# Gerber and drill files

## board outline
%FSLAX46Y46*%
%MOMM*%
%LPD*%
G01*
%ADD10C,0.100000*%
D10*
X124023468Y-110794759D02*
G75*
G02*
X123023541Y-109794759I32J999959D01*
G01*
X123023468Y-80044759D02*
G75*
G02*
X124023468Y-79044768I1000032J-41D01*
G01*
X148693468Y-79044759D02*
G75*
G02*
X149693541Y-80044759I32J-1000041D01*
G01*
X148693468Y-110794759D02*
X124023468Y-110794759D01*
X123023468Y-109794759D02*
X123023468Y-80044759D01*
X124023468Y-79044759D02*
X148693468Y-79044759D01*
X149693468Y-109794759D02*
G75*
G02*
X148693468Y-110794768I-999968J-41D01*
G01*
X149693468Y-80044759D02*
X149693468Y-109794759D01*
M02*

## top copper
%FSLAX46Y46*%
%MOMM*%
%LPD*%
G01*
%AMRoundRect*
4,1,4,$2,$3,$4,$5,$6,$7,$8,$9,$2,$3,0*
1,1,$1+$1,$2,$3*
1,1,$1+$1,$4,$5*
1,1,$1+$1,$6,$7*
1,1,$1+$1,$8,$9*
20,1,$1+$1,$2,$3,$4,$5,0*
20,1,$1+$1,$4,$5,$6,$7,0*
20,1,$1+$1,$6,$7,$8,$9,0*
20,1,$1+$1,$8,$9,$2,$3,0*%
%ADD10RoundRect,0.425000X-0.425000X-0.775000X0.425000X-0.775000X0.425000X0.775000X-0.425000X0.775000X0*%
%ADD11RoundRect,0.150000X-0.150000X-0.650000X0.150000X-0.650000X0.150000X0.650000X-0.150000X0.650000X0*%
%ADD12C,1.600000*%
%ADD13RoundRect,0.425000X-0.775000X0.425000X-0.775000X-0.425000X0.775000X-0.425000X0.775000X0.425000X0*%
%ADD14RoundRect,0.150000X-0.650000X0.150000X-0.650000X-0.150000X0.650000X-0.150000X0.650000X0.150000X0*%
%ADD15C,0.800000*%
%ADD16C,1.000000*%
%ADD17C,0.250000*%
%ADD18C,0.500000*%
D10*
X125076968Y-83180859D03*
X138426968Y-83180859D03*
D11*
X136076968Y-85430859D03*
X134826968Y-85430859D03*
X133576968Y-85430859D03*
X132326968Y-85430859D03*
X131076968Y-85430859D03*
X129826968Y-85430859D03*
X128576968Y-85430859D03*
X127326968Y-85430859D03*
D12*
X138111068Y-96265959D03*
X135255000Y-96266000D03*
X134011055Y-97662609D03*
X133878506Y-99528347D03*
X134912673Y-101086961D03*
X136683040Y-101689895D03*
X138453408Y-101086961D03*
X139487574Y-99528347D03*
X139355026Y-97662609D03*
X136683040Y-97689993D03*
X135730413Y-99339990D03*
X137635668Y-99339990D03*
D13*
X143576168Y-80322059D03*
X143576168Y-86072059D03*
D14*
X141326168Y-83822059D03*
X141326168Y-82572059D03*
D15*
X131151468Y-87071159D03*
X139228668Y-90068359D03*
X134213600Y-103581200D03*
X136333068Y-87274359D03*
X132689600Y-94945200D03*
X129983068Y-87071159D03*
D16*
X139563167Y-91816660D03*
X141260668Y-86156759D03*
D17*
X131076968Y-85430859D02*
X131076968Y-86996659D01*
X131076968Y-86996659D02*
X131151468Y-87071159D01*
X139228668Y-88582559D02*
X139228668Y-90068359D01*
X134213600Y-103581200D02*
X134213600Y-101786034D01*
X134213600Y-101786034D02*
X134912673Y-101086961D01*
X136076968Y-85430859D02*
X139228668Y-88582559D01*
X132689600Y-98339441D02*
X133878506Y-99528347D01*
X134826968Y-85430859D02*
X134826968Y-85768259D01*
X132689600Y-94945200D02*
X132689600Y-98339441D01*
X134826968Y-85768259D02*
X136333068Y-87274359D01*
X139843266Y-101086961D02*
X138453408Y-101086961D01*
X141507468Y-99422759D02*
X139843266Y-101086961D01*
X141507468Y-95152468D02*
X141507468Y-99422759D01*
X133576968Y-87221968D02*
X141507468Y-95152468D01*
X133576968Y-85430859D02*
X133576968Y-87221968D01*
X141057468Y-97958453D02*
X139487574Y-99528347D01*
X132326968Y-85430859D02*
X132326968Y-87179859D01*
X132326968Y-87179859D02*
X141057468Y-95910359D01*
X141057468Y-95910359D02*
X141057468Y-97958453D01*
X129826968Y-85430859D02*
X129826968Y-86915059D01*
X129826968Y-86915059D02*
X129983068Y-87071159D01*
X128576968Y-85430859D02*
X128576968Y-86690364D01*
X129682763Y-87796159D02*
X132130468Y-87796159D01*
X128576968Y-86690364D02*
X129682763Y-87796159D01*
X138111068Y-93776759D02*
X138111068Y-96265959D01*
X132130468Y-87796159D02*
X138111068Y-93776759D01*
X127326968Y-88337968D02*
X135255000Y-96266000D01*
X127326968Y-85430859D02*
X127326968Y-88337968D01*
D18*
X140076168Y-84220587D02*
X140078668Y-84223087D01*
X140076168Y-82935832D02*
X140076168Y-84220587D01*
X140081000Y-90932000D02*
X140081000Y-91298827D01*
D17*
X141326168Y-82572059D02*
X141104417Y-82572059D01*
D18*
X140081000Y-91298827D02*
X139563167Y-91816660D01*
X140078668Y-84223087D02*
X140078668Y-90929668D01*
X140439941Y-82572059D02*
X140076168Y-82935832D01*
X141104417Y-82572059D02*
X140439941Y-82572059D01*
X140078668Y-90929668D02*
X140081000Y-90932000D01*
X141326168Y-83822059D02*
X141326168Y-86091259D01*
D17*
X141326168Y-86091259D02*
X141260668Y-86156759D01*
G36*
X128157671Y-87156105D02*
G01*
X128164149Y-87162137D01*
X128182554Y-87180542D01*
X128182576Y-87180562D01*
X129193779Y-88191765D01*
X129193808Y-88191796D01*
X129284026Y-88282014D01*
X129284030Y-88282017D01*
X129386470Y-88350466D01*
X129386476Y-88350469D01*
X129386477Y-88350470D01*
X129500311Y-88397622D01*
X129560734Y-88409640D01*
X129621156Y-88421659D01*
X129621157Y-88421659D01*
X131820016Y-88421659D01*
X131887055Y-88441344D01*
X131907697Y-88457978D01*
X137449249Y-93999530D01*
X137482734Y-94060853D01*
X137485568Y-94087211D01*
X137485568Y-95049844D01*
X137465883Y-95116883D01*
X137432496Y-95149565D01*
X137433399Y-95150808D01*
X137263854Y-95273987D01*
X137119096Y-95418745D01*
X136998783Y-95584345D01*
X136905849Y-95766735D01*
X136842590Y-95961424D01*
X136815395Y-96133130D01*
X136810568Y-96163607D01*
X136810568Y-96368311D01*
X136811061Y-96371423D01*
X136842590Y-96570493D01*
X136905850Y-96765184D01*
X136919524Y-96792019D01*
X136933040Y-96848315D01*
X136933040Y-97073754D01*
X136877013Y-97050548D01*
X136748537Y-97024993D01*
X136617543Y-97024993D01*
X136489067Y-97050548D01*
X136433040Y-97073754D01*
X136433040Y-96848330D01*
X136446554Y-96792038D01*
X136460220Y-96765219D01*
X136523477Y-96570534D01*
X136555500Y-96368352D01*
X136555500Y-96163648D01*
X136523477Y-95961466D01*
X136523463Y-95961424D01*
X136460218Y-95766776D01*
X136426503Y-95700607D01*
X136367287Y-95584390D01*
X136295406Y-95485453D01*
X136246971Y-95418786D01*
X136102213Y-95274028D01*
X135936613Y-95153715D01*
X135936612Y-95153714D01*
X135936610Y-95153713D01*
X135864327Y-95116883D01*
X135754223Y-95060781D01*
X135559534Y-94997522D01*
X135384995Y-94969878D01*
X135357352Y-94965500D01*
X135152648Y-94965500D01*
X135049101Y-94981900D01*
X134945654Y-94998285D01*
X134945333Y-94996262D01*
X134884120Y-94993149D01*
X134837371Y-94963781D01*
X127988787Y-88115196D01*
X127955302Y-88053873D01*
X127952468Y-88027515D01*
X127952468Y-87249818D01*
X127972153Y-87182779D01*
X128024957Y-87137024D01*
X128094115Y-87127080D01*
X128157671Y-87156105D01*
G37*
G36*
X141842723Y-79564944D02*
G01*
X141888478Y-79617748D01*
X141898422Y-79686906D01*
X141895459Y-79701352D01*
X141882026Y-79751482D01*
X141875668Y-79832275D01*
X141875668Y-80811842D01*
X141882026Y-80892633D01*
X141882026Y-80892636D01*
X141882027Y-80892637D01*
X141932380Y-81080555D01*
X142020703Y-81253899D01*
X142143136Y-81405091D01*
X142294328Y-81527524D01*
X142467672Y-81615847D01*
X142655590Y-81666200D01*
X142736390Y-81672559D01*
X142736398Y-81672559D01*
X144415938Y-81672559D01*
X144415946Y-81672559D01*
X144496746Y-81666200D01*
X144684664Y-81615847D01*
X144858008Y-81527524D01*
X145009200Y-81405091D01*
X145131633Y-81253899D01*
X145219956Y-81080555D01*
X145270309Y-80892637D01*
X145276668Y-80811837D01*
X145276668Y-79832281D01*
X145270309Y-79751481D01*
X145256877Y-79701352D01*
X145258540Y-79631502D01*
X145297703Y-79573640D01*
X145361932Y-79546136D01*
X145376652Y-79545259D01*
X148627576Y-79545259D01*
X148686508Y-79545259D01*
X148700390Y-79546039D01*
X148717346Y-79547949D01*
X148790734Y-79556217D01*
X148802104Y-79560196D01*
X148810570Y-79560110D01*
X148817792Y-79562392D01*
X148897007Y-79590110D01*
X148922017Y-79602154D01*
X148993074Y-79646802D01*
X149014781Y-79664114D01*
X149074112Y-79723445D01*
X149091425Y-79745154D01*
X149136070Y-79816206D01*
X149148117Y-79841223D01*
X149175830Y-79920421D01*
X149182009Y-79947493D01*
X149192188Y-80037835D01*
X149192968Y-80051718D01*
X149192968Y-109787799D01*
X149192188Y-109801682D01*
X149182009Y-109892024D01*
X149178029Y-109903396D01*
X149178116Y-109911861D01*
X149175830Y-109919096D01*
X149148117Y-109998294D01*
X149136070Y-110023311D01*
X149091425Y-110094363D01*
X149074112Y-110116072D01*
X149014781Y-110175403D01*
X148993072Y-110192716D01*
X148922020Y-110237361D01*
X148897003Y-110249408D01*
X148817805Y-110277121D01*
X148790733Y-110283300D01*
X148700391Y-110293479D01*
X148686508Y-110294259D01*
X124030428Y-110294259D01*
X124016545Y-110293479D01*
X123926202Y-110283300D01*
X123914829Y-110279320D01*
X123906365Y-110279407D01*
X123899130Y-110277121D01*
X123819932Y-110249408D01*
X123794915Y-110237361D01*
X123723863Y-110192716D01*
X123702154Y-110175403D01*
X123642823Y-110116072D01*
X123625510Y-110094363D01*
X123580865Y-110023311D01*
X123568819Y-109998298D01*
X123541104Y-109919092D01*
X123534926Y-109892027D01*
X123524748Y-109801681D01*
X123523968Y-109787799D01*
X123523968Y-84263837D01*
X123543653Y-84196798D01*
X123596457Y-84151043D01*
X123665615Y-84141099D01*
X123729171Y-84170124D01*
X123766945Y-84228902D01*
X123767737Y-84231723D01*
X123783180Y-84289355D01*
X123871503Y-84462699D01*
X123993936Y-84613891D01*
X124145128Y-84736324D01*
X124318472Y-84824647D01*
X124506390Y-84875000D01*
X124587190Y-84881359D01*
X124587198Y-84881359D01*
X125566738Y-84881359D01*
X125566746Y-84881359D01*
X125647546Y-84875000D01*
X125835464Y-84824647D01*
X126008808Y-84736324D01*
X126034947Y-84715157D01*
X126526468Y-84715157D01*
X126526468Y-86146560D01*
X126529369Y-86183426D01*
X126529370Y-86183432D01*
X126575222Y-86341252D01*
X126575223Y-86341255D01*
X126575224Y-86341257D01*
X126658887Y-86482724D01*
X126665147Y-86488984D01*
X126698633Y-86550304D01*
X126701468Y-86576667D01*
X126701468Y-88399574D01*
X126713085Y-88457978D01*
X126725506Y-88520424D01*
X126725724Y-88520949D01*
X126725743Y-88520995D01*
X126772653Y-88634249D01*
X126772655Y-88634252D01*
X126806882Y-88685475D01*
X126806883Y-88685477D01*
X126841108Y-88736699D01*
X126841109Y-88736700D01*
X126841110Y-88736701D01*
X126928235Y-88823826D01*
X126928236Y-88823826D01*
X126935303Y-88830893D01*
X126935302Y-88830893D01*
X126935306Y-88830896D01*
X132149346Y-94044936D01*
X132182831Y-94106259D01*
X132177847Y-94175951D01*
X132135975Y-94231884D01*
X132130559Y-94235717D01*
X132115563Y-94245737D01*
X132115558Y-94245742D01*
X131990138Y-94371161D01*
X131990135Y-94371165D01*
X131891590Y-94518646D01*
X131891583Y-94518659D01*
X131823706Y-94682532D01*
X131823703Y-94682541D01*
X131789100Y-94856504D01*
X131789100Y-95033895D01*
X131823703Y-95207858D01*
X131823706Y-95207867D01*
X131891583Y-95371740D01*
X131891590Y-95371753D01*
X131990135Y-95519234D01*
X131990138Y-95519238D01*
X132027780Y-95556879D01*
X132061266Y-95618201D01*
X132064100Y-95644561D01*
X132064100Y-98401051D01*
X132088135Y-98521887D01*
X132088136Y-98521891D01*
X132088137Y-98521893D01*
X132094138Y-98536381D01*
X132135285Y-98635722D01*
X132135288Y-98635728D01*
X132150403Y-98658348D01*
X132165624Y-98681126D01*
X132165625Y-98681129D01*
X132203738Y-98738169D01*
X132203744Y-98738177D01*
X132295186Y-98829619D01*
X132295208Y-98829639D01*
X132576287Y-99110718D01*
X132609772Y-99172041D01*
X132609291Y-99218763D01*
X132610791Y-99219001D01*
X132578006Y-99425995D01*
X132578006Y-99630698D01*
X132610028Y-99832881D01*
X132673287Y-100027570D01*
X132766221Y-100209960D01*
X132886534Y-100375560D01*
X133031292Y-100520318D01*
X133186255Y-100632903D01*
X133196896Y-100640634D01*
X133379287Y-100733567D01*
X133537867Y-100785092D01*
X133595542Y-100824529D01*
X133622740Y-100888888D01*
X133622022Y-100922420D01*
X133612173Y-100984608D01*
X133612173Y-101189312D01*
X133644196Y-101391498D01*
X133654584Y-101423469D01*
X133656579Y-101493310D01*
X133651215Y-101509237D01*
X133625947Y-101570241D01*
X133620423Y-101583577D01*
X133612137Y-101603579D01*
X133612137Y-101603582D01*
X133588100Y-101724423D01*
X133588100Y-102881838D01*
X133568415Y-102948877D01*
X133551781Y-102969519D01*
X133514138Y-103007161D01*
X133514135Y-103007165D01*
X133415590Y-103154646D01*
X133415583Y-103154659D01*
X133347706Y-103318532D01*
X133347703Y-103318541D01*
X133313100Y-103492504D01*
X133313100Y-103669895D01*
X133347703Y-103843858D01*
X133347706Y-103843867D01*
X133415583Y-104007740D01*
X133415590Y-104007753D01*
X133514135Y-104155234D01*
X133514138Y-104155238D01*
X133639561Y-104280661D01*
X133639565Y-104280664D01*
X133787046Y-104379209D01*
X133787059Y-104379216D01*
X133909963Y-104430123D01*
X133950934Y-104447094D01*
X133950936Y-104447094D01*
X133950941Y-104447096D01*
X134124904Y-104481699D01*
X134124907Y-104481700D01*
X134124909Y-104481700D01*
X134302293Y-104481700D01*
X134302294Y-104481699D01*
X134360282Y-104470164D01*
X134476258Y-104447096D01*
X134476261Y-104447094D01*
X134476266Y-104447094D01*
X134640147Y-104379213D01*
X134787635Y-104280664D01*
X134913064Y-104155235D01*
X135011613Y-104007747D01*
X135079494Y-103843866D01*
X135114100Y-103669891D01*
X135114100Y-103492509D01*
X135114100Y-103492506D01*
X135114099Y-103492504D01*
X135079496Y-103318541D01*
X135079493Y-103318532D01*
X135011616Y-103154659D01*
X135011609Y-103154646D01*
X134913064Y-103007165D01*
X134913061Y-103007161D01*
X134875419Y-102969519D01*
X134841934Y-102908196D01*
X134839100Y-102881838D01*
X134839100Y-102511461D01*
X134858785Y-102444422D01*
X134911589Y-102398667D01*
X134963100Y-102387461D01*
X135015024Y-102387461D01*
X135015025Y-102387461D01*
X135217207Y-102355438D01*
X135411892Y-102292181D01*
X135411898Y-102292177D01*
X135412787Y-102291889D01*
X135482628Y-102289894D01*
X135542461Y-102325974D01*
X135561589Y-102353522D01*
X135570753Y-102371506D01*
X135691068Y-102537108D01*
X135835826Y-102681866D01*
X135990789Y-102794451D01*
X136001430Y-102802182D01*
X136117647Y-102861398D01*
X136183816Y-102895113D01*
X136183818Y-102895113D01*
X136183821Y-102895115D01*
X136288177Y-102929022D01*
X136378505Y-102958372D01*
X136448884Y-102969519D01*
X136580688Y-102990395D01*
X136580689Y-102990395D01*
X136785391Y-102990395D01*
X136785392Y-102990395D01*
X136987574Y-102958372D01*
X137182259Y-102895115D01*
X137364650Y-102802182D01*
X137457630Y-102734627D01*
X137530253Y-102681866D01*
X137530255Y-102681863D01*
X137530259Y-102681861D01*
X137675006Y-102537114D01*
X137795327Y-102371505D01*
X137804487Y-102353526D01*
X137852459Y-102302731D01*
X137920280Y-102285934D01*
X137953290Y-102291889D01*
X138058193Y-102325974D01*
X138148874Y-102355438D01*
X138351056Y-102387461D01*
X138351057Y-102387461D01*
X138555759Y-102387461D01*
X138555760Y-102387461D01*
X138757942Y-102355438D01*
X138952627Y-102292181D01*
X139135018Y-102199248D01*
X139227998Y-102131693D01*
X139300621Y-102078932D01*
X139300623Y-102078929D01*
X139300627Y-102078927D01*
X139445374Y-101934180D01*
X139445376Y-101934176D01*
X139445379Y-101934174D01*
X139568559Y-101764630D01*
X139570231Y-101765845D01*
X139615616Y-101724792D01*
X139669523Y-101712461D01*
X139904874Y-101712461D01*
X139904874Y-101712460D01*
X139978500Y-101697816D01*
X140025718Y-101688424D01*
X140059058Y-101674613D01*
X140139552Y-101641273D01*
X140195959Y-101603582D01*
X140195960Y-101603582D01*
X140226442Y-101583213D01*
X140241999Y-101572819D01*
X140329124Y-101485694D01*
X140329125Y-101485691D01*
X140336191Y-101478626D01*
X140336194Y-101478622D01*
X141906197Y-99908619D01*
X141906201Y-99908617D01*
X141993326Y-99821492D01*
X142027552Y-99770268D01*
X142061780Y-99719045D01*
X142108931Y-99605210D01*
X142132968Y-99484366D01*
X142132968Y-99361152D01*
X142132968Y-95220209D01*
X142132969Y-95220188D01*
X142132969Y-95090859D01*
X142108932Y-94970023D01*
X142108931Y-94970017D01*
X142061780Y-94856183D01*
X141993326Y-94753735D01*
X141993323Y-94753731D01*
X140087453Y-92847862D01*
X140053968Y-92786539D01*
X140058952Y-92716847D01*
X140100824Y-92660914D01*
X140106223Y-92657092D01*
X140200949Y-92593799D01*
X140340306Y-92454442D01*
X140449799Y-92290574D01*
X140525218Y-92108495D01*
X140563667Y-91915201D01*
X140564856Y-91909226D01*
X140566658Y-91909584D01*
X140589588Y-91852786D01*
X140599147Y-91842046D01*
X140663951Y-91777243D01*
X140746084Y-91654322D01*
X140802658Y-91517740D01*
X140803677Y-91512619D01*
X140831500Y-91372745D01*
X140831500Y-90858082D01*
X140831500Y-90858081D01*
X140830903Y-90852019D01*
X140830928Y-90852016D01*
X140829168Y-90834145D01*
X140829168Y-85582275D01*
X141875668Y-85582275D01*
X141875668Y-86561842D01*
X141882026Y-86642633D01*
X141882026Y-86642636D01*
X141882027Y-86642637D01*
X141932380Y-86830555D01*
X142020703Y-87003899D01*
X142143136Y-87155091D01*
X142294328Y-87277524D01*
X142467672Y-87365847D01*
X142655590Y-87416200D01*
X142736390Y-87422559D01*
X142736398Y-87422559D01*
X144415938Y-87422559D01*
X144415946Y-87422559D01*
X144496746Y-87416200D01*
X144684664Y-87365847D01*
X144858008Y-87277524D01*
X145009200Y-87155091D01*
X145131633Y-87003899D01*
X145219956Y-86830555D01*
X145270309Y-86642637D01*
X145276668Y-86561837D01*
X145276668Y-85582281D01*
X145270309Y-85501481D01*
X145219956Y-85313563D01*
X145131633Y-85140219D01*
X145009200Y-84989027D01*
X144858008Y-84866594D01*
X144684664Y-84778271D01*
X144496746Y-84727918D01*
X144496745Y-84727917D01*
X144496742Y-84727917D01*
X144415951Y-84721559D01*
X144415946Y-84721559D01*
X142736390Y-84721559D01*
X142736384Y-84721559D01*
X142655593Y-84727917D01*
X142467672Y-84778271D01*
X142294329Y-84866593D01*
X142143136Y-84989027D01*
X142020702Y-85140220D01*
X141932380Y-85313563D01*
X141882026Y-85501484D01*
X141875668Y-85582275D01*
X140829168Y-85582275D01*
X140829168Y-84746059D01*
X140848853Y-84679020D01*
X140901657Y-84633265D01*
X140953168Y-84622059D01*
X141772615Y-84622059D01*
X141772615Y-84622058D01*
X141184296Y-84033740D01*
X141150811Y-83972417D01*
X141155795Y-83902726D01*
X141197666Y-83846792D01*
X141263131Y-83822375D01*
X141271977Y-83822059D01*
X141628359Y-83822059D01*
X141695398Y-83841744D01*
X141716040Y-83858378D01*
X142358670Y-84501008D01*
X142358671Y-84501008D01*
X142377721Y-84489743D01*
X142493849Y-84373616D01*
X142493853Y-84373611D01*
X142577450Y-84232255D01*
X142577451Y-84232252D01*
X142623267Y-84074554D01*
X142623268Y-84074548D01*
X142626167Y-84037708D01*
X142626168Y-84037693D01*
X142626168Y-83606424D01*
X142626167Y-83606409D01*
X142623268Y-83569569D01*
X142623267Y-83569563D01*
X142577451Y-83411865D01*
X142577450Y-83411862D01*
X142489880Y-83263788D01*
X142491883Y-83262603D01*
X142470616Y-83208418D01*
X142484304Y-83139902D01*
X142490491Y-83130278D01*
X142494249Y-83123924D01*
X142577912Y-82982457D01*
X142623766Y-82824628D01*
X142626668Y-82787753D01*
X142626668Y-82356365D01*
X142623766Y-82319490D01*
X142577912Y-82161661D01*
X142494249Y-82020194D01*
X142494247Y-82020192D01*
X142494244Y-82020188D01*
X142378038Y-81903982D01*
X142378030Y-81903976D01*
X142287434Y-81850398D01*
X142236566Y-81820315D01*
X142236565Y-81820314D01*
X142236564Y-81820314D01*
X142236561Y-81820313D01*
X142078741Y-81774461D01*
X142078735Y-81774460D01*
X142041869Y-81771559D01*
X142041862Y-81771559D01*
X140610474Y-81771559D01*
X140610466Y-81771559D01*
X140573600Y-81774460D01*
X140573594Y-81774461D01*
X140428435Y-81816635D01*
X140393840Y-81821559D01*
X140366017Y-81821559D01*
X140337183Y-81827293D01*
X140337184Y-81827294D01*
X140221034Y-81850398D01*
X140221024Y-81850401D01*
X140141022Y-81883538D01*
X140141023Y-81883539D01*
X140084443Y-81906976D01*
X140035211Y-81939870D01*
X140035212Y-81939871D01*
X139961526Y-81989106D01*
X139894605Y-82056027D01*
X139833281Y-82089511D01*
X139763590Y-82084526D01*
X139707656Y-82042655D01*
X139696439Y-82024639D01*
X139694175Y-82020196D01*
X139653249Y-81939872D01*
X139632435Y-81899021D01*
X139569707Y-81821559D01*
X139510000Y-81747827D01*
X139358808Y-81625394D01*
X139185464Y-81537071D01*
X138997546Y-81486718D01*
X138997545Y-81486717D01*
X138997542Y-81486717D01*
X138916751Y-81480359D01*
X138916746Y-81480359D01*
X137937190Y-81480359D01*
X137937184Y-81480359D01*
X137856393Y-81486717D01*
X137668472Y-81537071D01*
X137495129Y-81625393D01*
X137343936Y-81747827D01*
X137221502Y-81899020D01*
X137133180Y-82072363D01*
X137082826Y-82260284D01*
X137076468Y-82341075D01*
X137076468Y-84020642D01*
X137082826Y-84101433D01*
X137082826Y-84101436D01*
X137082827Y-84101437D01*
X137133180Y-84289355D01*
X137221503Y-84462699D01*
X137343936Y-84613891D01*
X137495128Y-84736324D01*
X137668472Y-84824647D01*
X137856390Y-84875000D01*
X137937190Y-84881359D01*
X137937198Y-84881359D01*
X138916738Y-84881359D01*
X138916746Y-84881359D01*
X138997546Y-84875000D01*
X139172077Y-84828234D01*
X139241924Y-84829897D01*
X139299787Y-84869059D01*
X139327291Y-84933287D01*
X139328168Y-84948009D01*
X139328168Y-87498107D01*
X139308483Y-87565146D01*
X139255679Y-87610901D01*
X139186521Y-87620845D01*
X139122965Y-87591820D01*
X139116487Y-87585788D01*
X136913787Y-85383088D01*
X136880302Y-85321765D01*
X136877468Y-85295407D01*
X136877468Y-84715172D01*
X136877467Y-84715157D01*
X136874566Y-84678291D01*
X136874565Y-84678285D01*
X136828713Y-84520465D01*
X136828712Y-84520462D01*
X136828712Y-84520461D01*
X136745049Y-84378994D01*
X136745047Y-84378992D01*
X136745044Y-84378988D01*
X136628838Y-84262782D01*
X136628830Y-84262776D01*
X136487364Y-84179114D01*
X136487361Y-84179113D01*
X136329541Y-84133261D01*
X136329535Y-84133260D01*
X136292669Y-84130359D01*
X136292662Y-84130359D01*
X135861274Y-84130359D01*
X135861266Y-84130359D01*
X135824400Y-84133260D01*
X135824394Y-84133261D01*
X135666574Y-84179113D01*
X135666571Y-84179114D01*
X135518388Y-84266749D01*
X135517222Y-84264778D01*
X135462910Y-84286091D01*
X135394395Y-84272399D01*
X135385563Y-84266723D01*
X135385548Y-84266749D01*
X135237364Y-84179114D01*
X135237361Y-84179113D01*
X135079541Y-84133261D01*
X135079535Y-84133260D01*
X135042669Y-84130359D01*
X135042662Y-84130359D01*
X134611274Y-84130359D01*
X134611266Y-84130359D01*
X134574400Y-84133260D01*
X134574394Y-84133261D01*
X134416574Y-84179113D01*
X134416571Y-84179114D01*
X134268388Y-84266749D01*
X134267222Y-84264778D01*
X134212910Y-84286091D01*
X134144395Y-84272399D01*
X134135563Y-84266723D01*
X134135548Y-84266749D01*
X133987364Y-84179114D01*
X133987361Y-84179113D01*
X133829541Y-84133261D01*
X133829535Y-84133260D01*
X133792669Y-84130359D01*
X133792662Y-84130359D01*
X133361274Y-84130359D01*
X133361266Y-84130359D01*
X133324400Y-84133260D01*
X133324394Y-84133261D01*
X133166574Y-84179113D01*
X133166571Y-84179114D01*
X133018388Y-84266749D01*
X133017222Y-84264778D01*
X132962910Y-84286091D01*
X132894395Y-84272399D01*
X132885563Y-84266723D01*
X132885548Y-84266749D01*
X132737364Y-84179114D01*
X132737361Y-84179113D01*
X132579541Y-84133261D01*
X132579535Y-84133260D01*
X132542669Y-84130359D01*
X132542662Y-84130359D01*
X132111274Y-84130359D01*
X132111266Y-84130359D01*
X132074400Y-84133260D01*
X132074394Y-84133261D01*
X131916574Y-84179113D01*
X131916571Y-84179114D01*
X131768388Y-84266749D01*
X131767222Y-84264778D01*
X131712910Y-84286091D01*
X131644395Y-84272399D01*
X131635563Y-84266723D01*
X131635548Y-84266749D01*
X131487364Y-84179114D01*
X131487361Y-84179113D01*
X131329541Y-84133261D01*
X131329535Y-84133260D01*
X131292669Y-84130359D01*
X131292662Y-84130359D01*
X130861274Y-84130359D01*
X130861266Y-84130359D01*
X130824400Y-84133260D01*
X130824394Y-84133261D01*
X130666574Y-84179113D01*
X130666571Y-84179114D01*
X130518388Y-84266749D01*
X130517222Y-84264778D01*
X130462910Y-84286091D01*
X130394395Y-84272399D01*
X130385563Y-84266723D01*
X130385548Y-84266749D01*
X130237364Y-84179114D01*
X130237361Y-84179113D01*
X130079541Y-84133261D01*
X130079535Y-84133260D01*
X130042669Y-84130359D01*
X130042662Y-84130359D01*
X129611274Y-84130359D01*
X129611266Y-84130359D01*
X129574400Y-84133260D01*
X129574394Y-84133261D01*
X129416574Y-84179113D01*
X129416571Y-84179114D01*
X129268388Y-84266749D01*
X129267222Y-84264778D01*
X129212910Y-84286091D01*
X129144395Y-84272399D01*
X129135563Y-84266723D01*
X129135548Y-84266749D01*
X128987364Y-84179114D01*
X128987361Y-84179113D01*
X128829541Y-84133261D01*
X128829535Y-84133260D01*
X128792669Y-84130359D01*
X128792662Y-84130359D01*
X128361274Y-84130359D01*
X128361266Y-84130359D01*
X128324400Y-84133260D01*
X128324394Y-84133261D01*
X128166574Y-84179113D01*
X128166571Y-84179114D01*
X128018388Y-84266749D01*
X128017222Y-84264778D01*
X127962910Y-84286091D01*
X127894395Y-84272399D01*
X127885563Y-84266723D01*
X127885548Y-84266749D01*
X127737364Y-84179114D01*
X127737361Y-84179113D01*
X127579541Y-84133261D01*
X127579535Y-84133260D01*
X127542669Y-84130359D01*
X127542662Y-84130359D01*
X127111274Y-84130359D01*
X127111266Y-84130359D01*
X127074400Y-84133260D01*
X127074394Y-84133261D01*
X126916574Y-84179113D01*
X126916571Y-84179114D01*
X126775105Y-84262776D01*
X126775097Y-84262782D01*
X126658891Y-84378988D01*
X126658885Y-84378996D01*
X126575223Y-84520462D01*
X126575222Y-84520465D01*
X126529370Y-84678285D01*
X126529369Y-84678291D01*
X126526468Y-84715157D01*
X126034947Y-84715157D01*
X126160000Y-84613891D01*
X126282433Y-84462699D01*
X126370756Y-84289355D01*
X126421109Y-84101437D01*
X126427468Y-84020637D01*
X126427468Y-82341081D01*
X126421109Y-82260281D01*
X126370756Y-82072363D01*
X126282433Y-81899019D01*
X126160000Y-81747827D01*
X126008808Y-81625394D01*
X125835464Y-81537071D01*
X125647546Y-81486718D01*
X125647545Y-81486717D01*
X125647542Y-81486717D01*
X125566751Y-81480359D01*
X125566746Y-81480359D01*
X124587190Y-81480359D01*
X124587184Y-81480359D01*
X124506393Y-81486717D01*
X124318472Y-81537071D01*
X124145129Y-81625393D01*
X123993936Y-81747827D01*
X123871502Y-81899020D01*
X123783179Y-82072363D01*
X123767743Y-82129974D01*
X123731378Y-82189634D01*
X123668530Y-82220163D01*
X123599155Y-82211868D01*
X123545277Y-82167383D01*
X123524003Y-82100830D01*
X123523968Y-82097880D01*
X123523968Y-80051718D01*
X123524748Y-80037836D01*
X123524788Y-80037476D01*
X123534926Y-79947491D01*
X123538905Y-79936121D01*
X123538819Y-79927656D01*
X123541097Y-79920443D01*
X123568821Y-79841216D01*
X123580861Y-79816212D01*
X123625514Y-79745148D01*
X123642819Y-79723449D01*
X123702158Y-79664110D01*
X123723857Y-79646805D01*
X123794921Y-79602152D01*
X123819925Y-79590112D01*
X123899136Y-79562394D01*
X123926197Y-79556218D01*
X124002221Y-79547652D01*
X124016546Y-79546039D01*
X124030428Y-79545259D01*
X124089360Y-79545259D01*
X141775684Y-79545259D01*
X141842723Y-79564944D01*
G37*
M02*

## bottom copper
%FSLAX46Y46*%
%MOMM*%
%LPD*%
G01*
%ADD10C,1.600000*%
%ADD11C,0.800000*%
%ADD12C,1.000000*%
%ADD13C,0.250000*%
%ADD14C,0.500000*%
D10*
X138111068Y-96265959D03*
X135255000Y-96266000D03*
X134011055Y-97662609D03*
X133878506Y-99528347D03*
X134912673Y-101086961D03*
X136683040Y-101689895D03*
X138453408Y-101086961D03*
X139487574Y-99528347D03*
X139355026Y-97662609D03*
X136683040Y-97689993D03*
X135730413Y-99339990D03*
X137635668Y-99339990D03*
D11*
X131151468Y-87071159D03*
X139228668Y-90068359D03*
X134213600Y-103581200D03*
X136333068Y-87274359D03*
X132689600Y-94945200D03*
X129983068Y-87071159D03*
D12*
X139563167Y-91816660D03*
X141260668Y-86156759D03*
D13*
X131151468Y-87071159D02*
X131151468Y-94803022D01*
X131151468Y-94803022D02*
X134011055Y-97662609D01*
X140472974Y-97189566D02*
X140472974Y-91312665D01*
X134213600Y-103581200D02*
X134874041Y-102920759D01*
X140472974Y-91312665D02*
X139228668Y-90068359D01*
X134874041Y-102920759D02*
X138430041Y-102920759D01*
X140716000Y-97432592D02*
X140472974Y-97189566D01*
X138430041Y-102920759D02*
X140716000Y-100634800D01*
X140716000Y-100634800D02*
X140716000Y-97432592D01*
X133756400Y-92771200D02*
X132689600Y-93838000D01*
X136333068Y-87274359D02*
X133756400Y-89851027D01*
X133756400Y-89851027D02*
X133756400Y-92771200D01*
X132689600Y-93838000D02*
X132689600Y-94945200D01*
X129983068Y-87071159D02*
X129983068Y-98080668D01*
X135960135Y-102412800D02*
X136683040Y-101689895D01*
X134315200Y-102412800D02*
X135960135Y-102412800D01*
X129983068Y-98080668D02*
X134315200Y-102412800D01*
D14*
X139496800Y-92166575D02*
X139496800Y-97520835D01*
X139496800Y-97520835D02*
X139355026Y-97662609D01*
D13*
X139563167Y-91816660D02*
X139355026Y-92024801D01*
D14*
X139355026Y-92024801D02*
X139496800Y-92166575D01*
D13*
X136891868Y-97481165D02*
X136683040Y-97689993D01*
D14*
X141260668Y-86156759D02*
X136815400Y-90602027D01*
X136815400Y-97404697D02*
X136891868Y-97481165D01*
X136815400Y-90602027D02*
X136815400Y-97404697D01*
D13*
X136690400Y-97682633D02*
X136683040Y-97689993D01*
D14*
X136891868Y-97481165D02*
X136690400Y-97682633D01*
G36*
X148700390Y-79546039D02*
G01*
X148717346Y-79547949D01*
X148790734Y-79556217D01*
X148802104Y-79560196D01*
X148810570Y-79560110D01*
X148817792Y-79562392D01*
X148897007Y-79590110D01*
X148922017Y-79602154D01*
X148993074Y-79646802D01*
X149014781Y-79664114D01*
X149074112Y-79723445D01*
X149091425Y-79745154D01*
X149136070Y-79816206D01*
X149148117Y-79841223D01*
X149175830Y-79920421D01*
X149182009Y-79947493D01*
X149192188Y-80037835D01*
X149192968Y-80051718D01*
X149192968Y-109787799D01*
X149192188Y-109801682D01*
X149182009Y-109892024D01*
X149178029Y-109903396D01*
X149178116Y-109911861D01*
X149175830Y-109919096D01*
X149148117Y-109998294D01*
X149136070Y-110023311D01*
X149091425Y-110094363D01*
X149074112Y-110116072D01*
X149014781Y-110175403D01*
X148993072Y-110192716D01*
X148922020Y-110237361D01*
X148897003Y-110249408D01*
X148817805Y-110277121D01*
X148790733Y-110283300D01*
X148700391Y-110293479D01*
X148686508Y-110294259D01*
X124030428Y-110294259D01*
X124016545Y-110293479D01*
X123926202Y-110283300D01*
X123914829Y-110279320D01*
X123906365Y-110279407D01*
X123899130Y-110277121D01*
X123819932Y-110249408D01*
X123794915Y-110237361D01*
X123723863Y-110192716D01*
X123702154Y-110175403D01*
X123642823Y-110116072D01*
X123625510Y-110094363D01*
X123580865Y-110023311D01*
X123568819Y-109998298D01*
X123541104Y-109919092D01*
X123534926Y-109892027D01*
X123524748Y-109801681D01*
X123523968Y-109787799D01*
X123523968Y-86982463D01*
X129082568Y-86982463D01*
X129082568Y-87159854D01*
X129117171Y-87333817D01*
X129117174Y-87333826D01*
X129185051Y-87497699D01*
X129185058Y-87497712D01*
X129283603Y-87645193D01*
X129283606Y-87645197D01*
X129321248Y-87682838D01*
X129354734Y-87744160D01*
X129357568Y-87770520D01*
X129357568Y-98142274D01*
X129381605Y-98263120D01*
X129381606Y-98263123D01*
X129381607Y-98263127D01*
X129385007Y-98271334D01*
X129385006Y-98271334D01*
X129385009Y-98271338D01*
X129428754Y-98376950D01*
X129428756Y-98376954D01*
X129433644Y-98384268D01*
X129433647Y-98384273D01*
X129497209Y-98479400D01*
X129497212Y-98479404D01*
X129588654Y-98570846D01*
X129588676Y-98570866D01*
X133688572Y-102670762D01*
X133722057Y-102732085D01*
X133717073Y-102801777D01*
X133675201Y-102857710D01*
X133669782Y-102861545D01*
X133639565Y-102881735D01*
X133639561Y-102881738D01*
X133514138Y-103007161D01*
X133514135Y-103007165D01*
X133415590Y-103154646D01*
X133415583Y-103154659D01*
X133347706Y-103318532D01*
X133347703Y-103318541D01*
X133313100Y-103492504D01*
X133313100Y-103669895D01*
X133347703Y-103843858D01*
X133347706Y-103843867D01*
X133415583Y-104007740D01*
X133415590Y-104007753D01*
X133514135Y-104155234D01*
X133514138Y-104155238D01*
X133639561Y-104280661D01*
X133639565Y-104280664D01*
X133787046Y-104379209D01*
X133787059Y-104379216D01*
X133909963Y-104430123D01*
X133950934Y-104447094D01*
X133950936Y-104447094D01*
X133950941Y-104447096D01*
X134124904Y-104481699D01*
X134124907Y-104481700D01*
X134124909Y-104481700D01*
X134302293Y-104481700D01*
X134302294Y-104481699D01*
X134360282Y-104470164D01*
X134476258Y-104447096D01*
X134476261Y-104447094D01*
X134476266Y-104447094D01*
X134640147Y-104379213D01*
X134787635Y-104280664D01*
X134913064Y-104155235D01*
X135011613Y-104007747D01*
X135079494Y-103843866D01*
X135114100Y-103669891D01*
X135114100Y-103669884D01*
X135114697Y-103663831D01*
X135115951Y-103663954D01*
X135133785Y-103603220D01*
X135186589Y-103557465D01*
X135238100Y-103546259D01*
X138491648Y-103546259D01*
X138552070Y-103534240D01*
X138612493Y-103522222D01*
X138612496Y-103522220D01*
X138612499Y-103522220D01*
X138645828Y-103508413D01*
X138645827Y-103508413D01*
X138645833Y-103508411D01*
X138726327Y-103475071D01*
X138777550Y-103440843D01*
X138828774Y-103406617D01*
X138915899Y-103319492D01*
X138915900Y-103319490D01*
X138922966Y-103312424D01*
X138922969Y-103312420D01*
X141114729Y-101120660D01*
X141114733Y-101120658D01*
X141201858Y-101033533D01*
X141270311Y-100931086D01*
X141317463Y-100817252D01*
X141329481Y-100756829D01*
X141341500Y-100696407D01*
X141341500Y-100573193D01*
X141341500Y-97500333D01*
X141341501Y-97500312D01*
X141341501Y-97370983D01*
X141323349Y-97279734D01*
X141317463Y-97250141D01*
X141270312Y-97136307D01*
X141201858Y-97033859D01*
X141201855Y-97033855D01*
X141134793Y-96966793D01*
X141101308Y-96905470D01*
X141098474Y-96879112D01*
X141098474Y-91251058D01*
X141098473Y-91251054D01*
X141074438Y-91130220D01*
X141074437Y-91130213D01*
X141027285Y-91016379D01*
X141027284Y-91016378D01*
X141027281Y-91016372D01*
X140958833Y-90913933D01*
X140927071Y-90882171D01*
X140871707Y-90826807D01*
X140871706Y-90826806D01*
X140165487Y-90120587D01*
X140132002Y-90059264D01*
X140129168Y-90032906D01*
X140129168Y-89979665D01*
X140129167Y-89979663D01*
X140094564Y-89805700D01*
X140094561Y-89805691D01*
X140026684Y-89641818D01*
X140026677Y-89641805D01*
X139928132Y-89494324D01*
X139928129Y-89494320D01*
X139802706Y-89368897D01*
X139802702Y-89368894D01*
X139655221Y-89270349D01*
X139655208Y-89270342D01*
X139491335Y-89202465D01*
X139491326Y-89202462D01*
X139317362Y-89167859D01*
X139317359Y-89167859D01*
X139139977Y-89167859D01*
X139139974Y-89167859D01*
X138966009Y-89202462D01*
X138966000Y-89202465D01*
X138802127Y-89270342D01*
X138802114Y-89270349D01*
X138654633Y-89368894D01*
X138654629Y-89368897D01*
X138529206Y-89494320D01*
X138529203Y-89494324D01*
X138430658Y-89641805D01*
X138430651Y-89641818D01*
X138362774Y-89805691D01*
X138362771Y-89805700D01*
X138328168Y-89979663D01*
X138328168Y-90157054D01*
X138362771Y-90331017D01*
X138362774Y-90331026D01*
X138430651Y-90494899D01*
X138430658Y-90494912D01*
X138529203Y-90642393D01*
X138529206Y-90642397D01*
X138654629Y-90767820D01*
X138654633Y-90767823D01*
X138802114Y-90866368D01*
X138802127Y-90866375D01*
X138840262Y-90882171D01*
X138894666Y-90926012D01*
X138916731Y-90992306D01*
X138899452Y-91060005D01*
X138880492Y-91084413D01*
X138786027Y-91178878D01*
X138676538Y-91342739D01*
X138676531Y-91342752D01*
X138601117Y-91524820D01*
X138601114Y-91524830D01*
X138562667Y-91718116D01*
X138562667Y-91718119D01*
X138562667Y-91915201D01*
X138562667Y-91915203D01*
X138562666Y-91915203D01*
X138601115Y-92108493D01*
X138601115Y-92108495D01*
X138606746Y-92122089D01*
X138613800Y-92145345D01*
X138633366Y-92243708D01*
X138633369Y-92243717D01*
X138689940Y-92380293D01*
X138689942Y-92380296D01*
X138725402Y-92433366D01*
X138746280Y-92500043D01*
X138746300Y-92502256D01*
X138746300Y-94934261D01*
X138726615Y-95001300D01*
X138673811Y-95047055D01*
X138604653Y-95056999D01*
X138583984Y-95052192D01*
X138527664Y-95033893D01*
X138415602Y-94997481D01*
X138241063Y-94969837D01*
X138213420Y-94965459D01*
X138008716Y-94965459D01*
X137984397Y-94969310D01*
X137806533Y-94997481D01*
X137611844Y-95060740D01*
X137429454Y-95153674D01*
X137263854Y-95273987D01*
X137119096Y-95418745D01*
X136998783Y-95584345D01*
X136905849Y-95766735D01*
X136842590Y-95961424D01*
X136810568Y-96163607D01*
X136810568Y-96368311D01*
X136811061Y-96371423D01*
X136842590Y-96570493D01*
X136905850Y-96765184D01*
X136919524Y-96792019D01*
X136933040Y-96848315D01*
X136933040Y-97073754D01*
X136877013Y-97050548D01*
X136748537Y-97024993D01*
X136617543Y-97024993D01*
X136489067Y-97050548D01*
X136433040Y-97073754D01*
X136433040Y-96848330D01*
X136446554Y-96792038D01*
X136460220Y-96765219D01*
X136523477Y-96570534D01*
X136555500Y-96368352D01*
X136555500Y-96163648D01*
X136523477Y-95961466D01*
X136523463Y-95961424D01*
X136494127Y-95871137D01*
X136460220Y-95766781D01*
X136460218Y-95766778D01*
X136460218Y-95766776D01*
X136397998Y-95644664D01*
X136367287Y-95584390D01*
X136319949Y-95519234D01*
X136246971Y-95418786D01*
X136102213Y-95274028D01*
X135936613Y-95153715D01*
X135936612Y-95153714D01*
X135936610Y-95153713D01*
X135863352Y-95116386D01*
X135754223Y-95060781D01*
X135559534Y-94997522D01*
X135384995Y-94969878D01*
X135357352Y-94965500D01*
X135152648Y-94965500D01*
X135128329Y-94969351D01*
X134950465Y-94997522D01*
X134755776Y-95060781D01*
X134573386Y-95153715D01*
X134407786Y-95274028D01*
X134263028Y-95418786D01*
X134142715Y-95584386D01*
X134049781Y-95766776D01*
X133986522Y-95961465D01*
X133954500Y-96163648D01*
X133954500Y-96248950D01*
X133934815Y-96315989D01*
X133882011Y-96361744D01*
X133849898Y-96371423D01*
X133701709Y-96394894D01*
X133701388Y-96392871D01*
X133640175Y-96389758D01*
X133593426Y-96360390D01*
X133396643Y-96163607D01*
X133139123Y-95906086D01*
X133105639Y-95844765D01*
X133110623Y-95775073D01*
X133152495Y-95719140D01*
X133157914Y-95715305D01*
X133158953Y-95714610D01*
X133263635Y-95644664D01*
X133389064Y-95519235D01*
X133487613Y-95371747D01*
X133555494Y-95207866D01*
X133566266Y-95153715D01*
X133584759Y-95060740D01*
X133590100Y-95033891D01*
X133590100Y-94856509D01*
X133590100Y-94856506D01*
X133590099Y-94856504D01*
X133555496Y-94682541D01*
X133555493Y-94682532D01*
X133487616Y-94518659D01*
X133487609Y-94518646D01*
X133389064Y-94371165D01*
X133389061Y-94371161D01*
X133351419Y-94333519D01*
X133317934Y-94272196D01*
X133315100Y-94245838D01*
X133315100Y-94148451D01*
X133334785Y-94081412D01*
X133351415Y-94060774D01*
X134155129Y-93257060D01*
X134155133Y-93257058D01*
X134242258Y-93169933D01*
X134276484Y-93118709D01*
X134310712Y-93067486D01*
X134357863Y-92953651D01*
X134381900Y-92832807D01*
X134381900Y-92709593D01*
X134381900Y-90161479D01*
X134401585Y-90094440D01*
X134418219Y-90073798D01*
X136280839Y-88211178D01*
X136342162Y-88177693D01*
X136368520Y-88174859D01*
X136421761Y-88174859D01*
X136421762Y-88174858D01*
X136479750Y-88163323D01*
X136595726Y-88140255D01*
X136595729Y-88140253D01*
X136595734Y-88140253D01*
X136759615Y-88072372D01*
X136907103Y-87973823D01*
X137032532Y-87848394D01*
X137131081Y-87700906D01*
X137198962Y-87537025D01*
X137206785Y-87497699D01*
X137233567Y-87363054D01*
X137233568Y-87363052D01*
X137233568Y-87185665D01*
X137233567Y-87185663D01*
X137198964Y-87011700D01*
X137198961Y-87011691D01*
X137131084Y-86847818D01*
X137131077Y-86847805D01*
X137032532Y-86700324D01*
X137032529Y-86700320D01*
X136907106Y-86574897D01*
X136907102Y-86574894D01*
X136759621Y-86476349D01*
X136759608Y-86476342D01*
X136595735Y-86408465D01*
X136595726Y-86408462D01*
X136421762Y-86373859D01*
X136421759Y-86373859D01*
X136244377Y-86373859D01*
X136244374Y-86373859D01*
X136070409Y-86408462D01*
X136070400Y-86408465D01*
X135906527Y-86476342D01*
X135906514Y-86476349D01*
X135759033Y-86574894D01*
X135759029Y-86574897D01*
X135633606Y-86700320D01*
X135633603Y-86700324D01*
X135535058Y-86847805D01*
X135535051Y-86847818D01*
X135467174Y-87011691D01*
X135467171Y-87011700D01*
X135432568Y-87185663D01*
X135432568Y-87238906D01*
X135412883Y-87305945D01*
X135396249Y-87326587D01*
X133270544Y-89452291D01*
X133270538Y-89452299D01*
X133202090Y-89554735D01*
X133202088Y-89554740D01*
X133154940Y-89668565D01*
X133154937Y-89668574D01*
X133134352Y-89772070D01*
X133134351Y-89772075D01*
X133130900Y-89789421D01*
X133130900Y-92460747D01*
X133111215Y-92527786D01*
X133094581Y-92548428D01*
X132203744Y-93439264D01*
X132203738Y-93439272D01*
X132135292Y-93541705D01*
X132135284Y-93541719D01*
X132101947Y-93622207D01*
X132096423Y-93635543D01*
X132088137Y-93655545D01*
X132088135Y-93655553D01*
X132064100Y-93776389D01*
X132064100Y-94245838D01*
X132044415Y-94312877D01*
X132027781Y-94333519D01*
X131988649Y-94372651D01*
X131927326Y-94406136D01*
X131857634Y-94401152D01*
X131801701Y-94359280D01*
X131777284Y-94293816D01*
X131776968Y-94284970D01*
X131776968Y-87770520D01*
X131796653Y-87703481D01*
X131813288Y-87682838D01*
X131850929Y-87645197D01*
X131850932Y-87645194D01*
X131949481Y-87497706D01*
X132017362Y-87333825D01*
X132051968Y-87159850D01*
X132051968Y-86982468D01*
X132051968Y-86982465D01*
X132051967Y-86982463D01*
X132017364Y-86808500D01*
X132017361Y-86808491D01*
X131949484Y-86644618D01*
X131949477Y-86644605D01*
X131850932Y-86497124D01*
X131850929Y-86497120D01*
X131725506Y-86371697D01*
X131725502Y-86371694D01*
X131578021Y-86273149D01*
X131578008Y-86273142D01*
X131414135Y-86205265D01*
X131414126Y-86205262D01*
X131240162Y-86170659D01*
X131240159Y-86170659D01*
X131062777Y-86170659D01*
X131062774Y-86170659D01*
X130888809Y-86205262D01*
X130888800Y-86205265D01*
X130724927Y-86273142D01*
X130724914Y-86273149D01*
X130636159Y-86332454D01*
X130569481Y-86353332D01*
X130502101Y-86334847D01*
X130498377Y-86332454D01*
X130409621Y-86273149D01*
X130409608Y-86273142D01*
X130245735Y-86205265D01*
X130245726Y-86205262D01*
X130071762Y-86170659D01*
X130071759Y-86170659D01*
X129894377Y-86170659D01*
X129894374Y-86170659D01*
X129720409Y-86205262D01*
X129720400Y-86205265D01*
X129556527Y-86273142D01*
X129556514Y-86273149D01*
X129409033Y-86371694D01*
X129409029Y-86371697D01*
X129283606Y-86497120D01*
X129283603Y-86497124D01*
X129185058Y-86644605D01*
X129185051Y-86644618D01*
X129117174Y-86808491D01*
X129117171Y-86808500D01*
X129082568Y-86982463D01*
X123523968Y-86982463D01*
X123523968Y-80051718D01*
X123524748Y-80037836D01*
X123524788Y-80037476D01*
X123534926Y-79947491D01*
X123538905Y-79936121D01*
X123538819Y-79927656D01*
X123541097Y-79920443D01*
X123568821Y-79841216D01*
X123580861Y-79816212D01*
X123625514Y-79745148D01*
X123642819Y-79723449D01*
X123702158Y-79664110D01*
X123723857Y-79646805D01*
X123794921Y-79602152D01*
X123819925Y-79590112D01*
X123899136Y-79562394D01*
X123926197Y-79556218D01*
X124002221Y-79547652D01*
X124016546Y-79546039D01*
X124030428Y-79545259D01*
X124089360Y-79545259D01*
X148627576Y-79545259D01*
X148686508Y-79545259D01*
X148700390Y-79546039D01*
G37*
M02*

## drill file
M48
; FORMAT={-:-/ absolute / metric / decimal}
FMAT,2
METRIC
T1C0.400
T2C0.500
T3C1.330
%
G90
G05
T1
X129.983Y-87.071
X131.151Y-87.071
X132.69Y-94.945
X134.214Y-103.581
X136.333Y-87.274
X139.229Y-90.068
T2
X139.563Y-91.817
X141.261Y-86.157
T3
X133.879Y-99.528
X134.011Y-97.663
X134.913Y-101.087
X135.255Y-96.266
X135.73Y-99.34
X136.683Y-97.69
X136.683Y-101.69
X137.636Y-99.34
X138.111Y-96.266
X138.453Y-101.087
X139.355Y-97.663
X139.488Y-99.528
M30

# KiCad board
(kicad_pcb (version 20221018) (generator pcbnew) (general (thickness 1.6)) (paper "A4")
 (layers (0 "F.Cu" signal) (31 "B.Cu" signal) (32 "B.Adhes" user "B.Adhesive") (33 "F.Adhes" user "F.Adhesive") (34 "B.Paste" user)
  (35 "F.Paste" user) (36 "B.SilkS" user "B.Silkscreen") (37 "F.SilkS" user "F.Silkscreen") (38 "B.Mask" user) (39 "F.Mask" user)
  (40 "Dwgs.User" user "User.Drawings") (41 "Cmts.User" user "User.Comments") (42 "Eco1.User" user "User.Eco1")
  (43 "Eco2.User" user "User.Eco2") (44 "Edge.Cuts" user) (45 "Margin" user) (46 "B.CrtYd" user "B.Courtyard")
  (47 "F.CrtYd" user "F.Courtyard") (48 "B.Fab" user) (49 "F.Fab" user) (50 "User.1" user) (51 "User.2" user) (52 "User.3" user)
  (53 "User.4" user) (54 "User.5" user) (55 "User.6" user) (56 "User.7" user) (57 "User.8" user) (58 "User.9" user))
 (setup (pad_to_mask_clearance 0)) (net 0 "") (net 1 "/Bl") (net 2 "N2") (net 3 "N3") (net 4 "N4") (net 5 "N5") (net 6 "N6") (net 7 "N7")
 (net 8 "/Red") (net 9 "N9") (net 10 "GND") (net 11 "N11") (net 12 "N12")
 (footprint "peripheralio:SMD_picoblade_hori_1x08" (layer "F.Cu") (at 124.226968 86.230859)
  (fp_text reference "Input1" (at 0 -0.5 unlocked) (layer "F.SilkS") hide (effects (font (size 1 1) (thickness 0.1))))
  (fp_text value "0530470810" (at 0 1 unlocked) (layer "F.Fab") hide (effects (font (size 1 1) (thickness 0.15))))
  (pad "" smd roundrect (at 0.85 -3.05) (size 1.7 2.4) (layers "F.Cu" "F.Paste" "F.Mask") (roundrect_rratio 0.25) (thermal_bridge_angle 45))
  (pad "" smd roundrect (at 14.2 -3.05) (size 1.7 2.4) (layers "F.Cu" "F.Paste" "F.Mask") (roundrect_rratio 0.25) (thermal_bridge_angle 45))
  (pad "1" smd roundrect (at 11.85 -0.8) (size 0.6 1.6) (layers "F.Cu" "F.Paste" "F.Mask") (roundrect_rratio 0.25) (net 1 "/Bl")
   (thermal_bridge_angle 45))
  (pad "2" smd roundrect (at 10.6 -0.8) (size 0.6 1.6) (layers "F.Cu" "F.Paste" "F.Mask") (roundrect_rratio 0.25) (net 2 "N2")
   (thermal_bridge_angle 45))
  (pad "3" smd roundrect (at 9.35 -0.8) (size 0.6 1.6) (layers "F.Cu" "F.Paste" "F.Mask") (roundrect_rratio 0.25) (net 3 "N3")
   (thermal_bridge_angle 45))
  (pad "4" smd roundrect (at 8.1 -0.8) (size 0.6 1.6) (layers "F.Cu" "F.Paste" "F.Mask") (roundrect_rratio 0.25) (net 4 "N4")
   (thermal_bridge_angle 45))
  (pad "5" smd roundrect (at 6.85 -0.8) (size 0.6 1.6) (layers "F.Cu" "F.Paste" "F.Mask") (roundrect_rratio 0.25) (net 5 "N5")
   (thermal_bridge_angle 45))
  (pad "6" smd roundrect (at 5.6 -0.8) (size 0.6 1.6) (layers "F.Cu" "F.Paste" "F.Mask") (roundrect_rratio 0.25) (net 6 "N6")
   (thermal_bridge_angle 45))
  (pad "7" smd roundrect (at 4.35 -0.8) (size 0.6 1.6) (layers "F.Cu" "F.Paste" "F.Mask") (roundrect_rratio 0.25) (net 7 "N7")
   (thermal_bridge_angle 45))
  (pad "8" smd roundrect (at 3.1 -0.8) (size 0.6 1.6) (layers "F.Cu" "F.Paste" "F.Mask") (roundrect_rratio 0.25) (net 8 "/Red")
   (thermal_bridge_angle 45)))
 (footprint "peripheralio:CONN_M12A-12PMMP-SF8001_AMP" (layer "F.Cu") (at 138.111068 96.265959 45)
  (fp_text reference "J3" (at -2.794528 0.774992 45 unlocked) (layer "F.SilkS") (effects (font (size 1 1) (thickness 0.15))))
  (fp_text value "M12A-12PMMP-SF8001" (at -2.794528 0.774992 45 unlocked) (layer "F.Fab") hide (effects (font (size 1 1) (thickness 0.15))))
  (pad "1" thru_hole circle (at 0 0 45) (size 1.6 1.6) (drill 1.33) (layers "*.Cu" "*.Mask") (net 7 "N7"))
  (pad "2" thru_hole circle (at -2.019574 -2.019516 45) (size 1.6 1.6) (drill 1.33) (layers "*.Cu" "*.Mask") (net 8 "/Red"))
  (pad "3" thru_hole circle (at -3.886728 -1.911566 135) (size 1.6 1.6) (drill 1.33) (layers "*.Cu" "*.Mask") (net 5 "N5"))
  (pad "4" thru_hole circle (at -5.29973 -0.686016 45) (size 1.6 1.6) (drill 1.33) (layers "*.Cu" "*.Mask") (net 2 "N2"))
  (pad "5" thru_hole circle (at -5.67057 1.147356 45) (size 1.6 1.6) (drill 1.33) (layers "*.Cu" "*.Mask") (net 1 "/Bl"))
  (pad "6" thru_hole circle (at -4.84507 2.825534 45) (size 1.6 1.6) (drill 1.33) (layers "*.Cu" "*.Mask") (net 6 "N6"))
  (pad "7" thru_hole circle (at -3.166892 3.651034 45) (size 1.6 1.6) (drill 1.33) (layers "*.Cu" "*.Mask") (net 3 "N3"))
  (pad "8" thru_hole circle (at -1.33352 3.280194 45) (size 1.6 1.6) (drill 1.33) (layers "*.Cu" "*.Mask") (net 4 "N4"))
  (pad "9" thru_hole circle (at -0.10797 1.867192 45) (size 1.6 1.6) (drill 1.33) (layers "*.Cu" "*.Mask") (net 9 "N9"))
  (pad "10" thru_hole circle (at -2.016712 -0.002824 45) (size 1.6 1.6) (drill 1.33) (layers "*.Cu" "*.Mask") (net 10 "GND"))
  (pad "11" thru_hole circle (at -3.857046 0.490291 255) (size 1.6 1.6) (drill 1.33) (layers "*.Cu" "*.Mask") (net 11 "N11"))
  (pad "12" thru_hole circle (at -2.509827 1.83751 285) (size 1.6 1.6) (drill 1.33) (layers "*.Cu" "*.Mask") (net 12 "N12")))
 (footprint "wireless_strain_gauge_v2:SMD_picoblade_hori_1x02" (layer "F.Cu") (at 140.526168 79.472059 -90)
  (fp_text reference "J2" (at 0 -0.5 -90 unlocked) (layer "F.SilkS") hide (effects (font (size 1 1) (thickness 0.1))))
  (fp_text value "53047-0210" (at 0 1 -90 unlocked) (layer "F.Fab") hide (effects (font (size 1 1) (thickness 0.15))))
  (pad "" smd roundrect (at 0.85 -3.05 270) (size 1.7 2.4) (layers "F.Cu" "F.Paste" "F.Mask") (roundrect_rratio 0.25)
   (thermal_bridge_angle 45))
  (pad "" smd roundrect (at 6.6 -3.05 270) (size 1.7 2.4) (layers "F.Cu" "F.Paste" "F.Mask") (roundrect_rratio 0.25)
   (thermal_bridge_angle 45))
  (pad "1" smd roundrect (at 4.35 -0.8 270) (size 0.6 1.6) (layers "F.Cu" "F.Paste" "F.Mask") (roundrect_rratio 0.25) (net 10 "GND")
   (thermal_bridge_angle 45))
  (pad "2" smd roundrect (at 3.1 -0.8 270) (size 0.6 1.6) (layers "F.Cu" "F.Paste" "F.Mask") (roundrect_rratio 0.25) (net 9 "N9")
   (thermal_bridge_angle 45)))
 (gr_arc (start 124.023468 110.794759) (mid 123.316361 110.501866) (end 123.023468 109.794759) (stroke (width 0.1) (type default))
  (layer "Edge.Cuts"))
 (gr_arc (start 123.023468 80.044759) (mid 123.316361 79.337652) (end 124.023468 79.044759) (stroke (width 0.1) (type default))
  (layer "Edge.Cuts"))
 (gr_arc (start 148.693468 79.044759) (mid 149.400575 79.337652) (end 149.693468 80.044759) (stroke (width 0.1) (type default))
  (layer "Edge.Cuts"))
 (gr_line (start 148.693468 110.794759) (end 124.023468 110.794759) (stroke (width 0.1) (type default)) (layer "Edge.Cuts"))
 (gr_line (start 123.023468 109.794759) (end 123.023468 80.044759) (stroke (width 0.1) (type default)) (layer "Edge.Cuts"))
 (gr_line (start 124.023468 79.044759) (end 148.693468 79.044759) (stroke (width 0.1) (type default)) (layer "Edge.Cuts"))
 (gr_arc (start 149.693468 109.794759) (mid 149.400575 110.501866) (end 148.693468 110.794759) (stroke (width 0.1) (type default))
  (layer "Edge.Cuts"))
 (gr_line (start 149.693468 80.044759) (end 149.693468 109.794759) (stroke (width 0.1) (type default)) (layer "Edge.Cuts"))
 (segment (start 131.076968 85.430859) (end 131.076968 86.996659) (width 0.25) (layer "F.Cu") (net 5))
 (segment (start 131.076968 86.996659) (end 131.151468 87.071159) (width 0.25) (layer "F.Cu") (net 5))
 (via (at 131.151468 87.071159) (size 0.8) (drill 0.4) (layers "F.Cu" "B.Cu") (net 5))
 (segment (start 131.151468 87.071159) (end 131.151468 94.803022) (width 0.25) (layer "B.Cu") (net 5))
 (segment (start 131.151468 94.803022) (end 134.011055 97.662609) (width 0.25) (layer "B.Cu") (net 5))
 (segment (start 139.228668 88.582559) (end 139.228668 90.068359) (width 0.25) (layer "F.Cu") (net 1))
 (segment (start 134.2136 103.5812) (end 134.2136 101.786034) (width 0.25) (layer "F.Cu") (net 1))
 (segment (start 134.2136 101.786034) (end 134.912673 101.086961) (width 0.25) (layer "F.Cu") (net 1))
 (segment (start 136.076968 85.430859) (end 139.228668 88.582559) (width 0.25) (layer "F.Cu") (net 1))
 (via (at 139.228668 90.068359) (size 0.8) (drill 0.4) (layers "F.Cu" "B.Cu") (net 1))
 (via (at 134.2136 103.5812) (size 0.8) (drill 0.4) (layers "F.Cu" "B.Cu") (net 1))
 (segment (start 140.472974 97.189566) (end 140.472974 91.312665) (width 0.25) (layer "B.Cu") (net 1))
 (segment (start 134.2136 103.5812) (end 134.874041 102.920759) (width 0.25) (layer "B.Cu") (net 1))
 (segment (start 140.472974 91.312665) (end 139.228668 90.068359) (width 0.25) (layer "B.Cu") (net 1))
 (segment (start 134.874041 102.920759) (end 138.430041 102.920759) (width 0.25) (layer "B.Cu") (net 1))
 (segment (start 140.716 97.432592) (end 140.472974 97.189566) (width 0.25) (layer "B.Cu") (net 1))
 (segment (start 138.430041 102.920759) (end 140.716 100.6348) (width 0.25) (layer "B.Cu") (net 1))
 (segment (start 140.716 100.6348) (end 140.716 97.432592) (width 0.25) (layer "B.Cu") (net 1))
 (segment (start 132.6896 98.339441) (end 133.878506 99.528347) (width 0.25) (layer "F.Cu") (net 2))
 (segment (start 134.826968 85.430859) (end 134.826968 85.768259) (width 0.25) (layer "F.Cu") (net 2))
 (segment (start 132.6896 94.9452) (end 132.6896 98.339441) (width 0.25) (layer "F.Cu") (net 2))
 (segment (start 134.826968 85.768259) (end 136.333068 87.274359) (width 0.25) (layer "F.Cu") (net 2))
 (via (at 136.333068 87.274359) (size 0.8) (drill 0.4) (layers "F.Cu" "B.Cu") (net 2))
 (via (at 132.6896 94.9452) (size 0.8) (drill 0.4) (layers "F.Cu" "B.Cu") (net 2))
 (segment (start 133.7564 92.7712) (end 132.6896 93.838) (width 0.25) (layer "B.Cu") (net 2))
 (segment (start 136.333068 87.274359) (end 133.7564 89.851027) (width 0.25) (layer "B.Cu") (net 2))
 (segment (start 133.7564 89.851027) (end 133.7564 92.7712) (width 0.25) (layer "B.Cu") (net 2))
 (segment (start 132.6896 93.838) (end 132.6896 94.9452) (width 0.25) (layer "B.Cu") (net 2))
 (segment (start 139.843266 101.086961) (end 138.453408 101.086961) (width 0.25) (layer "F.Cu") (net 3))
 (segment (start 141.507468 99.422759) (end 139.843266 101.086961) (width 0.25) (layer "F.Cu") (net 3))
 (segment (start 141.507468 95.152468) (end 141.507468 99.422759) (width 0.25) (layer "F.Cu") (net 3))
 (segment (start 133.576968 87.221968) (end 141.507468 95.152468) (width 0.25) (layer "F.Cu") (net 3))
 (segment (start 133.576968 85.430859) (end 133.576968 87.221968) (width 0.25) (layer "F.Cu") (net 3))
 (segment (start 141.057468 97.958453) (end 139.487574 99.528347) (width 0.25) (layer "F.Cu") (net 4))
 (segment (start 132.326968 85.430859) (end 132.326968 87.179859) (width 0.25) (layer "F.Cu") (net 4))
 (segment (start 132.326968 87.179859) (end 141.057468 95.910359) (width 0.25) (layer "F.Cu") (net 4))
 (segment (start 141.057468 95.910359) (end 141.057468 97.958453) (width 0.25) (layer "F.Cu") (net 4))
 (segment (start 129.826968 85.430859) (end 129.826968 86.915059) (width 0.25) (layer "F.Cu") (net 6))
 (segment (start 129.826968 86.915059) (end 129.983068 87.071159) (width 0.25) (layer "F.Cu") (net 6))
 (via (at 129.983068 87.071159) (size 0.8) (drill 0.4) (layers "F.Cu" "B.Cu") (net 6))
 (segment (start 129.983068 87.071159) (end 129.983068 98.080668) (width 0.25) (layer "B.Cu") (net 6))
 (segment (start 135.960135 102.4128) (end 136.68304 101.689895) (width 0.25) (layer "B.Cu") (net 6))
 (segment (start 134.3152 102.4128) (end 135.960135 102.4128) (width 0.25) (layer "B.Cu") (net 6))
 (segment (start 129.983068 98.080668) (end 134.3152 102.4128) (width 0.25) (layer "B.Cu") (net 6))
 (segment (start 128.576968 85.430859) (end 128.576968 86.690364) (width 0.25) (layer "F.Cu") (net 7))
 (segment (start 129.682763 87.796159) (end 132.130468 87.796159) (width 0.25) (layer "F.Cu") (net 7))
 (segment (start 128.576968 86.690364) (end 129.682763 87.796159) (width 0.25) (layer "F.Cu") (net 7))
 (segment (start 138.111068 93.776759) (end 138.111068 96.265959) (width 0.25) (layer "F.Cu") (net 7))
 (segment (start 132.130468 87.796159) (end 138.111068 93.776759) (width 0.25) (layer "F.Cu") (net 7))
 (segment (start 127.326968 88.337968) (end 135.255 96.266) (width 0.25) (layer "F.Cu") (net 8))
 (segment (start 127.326968 85.430859) (end 127.326968 88.337968) (width 0.25) (layer "F.Cu") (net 8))
 (segment (start 140.076168 84.220587) (end 140.078668 84.223087) (width 0.5) (layer "F.Cu") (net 9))
 (segment (start 140.076168 82.935832) (end 140.076168 84.220587) (width 0.5) (layer "F.Cu") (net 9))
 (segment (start 140.081 90.932) (end 140.081 91.298827) (width 0.5) (layer "F.Cu") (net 9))
 (segment (start 141.326168 82.572059) (end 141.104417 82.572059) (width 0.25) (layer "F.Cu") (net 9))
 (segment (start 140.081 91.298827) (end 139.563167 91.81666) (width 0.5) (layer "F.Cu") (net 9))
 (segment (start 140.078668 84.223087) (end 140.078668 90.929668) (width 0.5) (layer "F.Cu") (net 9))
 (segment (start 140.439941 82.572059) (end 140.076168 82.935832) (width 0.5) (layer "F.Cu") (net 9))
 (segment (start 141.104417 82.572059) (end 140.439941 82.572059) (width 0.5) (layer "F.Cu") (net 9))
 (segment (start 140.078668 90.929668) (end 140.081 90.932) (width 0.5) (layer "F.Cu") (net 9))
 (via (at 139.563167 91.81666) (size 1) (drill 0.5) (layers "F.Cu" "B.Cu") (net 9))
 (segment (start 139.4968 92.166575) (end 139.4968 97.520835) (width 0.5) (layer "B.Cu") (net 9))
 (segment (start 139.4968 97.520835) (end 139.355026 97.662609) (width 0.5) (layer "B.Cu") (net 9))
 (segment (start 139.563167 91.81666) (end 139.355026 92.024801) (width 0.25) (layer "B.Cu") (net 9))
 (segment (start 139.355026 92.024801) (end 139.4968 92.166575) (width 0.5) (layer "B.Cu") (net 9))
 (segment (start 141.326168 83.822059) (end 141.326168 86.091259) (width 0.5) (layer "F.Cu") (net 10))
 (segment (start 141.326168 86.091259) (end 141.260668 86.156759) (width 0.25) (layer "F.Cu") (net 10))
 (via (at 141.260668 86.156759) (size 1) (drill 0.5) (layers "F.Cu" "B.Cu") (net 10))
 (segment (start 136.891868 97.481165) (end 136.68304 97.689993) (width 0.25) (layer "B.Cu") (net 10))
 (segment (start 141.260668 86.156759) (end 136.8154 90.602027) (width 0.5) (layer "B.Cu") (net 10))
 (segment (start 136.8154 97.404697) (end 136.891868 97.481165) (width 0.5) (layer "B.Cu") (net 10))
 (segment (start 136.8154 90.602027) (end 136.8154 97.404697) (width 0.5) (layer "B.Cu") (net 10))
 (segment (start 136.6904 97.682633) (end 136.68304 97.689993) (width 0.25) (layer "B.Cu") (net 10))
 (segment (start 136.891868 97.481165) (end 136.6904 97.682633) (width 0.5) (layer "B.Cu") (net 10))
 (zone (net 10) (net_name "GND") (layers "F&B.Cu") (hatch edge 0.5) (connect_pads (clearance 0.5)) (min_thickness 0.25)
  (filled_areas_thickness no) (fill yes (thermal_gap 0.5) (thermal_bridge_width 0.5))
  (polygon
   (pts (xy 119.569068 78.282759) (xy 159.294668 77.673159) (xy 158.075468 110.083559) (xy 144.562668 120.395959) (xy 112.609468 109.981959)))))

